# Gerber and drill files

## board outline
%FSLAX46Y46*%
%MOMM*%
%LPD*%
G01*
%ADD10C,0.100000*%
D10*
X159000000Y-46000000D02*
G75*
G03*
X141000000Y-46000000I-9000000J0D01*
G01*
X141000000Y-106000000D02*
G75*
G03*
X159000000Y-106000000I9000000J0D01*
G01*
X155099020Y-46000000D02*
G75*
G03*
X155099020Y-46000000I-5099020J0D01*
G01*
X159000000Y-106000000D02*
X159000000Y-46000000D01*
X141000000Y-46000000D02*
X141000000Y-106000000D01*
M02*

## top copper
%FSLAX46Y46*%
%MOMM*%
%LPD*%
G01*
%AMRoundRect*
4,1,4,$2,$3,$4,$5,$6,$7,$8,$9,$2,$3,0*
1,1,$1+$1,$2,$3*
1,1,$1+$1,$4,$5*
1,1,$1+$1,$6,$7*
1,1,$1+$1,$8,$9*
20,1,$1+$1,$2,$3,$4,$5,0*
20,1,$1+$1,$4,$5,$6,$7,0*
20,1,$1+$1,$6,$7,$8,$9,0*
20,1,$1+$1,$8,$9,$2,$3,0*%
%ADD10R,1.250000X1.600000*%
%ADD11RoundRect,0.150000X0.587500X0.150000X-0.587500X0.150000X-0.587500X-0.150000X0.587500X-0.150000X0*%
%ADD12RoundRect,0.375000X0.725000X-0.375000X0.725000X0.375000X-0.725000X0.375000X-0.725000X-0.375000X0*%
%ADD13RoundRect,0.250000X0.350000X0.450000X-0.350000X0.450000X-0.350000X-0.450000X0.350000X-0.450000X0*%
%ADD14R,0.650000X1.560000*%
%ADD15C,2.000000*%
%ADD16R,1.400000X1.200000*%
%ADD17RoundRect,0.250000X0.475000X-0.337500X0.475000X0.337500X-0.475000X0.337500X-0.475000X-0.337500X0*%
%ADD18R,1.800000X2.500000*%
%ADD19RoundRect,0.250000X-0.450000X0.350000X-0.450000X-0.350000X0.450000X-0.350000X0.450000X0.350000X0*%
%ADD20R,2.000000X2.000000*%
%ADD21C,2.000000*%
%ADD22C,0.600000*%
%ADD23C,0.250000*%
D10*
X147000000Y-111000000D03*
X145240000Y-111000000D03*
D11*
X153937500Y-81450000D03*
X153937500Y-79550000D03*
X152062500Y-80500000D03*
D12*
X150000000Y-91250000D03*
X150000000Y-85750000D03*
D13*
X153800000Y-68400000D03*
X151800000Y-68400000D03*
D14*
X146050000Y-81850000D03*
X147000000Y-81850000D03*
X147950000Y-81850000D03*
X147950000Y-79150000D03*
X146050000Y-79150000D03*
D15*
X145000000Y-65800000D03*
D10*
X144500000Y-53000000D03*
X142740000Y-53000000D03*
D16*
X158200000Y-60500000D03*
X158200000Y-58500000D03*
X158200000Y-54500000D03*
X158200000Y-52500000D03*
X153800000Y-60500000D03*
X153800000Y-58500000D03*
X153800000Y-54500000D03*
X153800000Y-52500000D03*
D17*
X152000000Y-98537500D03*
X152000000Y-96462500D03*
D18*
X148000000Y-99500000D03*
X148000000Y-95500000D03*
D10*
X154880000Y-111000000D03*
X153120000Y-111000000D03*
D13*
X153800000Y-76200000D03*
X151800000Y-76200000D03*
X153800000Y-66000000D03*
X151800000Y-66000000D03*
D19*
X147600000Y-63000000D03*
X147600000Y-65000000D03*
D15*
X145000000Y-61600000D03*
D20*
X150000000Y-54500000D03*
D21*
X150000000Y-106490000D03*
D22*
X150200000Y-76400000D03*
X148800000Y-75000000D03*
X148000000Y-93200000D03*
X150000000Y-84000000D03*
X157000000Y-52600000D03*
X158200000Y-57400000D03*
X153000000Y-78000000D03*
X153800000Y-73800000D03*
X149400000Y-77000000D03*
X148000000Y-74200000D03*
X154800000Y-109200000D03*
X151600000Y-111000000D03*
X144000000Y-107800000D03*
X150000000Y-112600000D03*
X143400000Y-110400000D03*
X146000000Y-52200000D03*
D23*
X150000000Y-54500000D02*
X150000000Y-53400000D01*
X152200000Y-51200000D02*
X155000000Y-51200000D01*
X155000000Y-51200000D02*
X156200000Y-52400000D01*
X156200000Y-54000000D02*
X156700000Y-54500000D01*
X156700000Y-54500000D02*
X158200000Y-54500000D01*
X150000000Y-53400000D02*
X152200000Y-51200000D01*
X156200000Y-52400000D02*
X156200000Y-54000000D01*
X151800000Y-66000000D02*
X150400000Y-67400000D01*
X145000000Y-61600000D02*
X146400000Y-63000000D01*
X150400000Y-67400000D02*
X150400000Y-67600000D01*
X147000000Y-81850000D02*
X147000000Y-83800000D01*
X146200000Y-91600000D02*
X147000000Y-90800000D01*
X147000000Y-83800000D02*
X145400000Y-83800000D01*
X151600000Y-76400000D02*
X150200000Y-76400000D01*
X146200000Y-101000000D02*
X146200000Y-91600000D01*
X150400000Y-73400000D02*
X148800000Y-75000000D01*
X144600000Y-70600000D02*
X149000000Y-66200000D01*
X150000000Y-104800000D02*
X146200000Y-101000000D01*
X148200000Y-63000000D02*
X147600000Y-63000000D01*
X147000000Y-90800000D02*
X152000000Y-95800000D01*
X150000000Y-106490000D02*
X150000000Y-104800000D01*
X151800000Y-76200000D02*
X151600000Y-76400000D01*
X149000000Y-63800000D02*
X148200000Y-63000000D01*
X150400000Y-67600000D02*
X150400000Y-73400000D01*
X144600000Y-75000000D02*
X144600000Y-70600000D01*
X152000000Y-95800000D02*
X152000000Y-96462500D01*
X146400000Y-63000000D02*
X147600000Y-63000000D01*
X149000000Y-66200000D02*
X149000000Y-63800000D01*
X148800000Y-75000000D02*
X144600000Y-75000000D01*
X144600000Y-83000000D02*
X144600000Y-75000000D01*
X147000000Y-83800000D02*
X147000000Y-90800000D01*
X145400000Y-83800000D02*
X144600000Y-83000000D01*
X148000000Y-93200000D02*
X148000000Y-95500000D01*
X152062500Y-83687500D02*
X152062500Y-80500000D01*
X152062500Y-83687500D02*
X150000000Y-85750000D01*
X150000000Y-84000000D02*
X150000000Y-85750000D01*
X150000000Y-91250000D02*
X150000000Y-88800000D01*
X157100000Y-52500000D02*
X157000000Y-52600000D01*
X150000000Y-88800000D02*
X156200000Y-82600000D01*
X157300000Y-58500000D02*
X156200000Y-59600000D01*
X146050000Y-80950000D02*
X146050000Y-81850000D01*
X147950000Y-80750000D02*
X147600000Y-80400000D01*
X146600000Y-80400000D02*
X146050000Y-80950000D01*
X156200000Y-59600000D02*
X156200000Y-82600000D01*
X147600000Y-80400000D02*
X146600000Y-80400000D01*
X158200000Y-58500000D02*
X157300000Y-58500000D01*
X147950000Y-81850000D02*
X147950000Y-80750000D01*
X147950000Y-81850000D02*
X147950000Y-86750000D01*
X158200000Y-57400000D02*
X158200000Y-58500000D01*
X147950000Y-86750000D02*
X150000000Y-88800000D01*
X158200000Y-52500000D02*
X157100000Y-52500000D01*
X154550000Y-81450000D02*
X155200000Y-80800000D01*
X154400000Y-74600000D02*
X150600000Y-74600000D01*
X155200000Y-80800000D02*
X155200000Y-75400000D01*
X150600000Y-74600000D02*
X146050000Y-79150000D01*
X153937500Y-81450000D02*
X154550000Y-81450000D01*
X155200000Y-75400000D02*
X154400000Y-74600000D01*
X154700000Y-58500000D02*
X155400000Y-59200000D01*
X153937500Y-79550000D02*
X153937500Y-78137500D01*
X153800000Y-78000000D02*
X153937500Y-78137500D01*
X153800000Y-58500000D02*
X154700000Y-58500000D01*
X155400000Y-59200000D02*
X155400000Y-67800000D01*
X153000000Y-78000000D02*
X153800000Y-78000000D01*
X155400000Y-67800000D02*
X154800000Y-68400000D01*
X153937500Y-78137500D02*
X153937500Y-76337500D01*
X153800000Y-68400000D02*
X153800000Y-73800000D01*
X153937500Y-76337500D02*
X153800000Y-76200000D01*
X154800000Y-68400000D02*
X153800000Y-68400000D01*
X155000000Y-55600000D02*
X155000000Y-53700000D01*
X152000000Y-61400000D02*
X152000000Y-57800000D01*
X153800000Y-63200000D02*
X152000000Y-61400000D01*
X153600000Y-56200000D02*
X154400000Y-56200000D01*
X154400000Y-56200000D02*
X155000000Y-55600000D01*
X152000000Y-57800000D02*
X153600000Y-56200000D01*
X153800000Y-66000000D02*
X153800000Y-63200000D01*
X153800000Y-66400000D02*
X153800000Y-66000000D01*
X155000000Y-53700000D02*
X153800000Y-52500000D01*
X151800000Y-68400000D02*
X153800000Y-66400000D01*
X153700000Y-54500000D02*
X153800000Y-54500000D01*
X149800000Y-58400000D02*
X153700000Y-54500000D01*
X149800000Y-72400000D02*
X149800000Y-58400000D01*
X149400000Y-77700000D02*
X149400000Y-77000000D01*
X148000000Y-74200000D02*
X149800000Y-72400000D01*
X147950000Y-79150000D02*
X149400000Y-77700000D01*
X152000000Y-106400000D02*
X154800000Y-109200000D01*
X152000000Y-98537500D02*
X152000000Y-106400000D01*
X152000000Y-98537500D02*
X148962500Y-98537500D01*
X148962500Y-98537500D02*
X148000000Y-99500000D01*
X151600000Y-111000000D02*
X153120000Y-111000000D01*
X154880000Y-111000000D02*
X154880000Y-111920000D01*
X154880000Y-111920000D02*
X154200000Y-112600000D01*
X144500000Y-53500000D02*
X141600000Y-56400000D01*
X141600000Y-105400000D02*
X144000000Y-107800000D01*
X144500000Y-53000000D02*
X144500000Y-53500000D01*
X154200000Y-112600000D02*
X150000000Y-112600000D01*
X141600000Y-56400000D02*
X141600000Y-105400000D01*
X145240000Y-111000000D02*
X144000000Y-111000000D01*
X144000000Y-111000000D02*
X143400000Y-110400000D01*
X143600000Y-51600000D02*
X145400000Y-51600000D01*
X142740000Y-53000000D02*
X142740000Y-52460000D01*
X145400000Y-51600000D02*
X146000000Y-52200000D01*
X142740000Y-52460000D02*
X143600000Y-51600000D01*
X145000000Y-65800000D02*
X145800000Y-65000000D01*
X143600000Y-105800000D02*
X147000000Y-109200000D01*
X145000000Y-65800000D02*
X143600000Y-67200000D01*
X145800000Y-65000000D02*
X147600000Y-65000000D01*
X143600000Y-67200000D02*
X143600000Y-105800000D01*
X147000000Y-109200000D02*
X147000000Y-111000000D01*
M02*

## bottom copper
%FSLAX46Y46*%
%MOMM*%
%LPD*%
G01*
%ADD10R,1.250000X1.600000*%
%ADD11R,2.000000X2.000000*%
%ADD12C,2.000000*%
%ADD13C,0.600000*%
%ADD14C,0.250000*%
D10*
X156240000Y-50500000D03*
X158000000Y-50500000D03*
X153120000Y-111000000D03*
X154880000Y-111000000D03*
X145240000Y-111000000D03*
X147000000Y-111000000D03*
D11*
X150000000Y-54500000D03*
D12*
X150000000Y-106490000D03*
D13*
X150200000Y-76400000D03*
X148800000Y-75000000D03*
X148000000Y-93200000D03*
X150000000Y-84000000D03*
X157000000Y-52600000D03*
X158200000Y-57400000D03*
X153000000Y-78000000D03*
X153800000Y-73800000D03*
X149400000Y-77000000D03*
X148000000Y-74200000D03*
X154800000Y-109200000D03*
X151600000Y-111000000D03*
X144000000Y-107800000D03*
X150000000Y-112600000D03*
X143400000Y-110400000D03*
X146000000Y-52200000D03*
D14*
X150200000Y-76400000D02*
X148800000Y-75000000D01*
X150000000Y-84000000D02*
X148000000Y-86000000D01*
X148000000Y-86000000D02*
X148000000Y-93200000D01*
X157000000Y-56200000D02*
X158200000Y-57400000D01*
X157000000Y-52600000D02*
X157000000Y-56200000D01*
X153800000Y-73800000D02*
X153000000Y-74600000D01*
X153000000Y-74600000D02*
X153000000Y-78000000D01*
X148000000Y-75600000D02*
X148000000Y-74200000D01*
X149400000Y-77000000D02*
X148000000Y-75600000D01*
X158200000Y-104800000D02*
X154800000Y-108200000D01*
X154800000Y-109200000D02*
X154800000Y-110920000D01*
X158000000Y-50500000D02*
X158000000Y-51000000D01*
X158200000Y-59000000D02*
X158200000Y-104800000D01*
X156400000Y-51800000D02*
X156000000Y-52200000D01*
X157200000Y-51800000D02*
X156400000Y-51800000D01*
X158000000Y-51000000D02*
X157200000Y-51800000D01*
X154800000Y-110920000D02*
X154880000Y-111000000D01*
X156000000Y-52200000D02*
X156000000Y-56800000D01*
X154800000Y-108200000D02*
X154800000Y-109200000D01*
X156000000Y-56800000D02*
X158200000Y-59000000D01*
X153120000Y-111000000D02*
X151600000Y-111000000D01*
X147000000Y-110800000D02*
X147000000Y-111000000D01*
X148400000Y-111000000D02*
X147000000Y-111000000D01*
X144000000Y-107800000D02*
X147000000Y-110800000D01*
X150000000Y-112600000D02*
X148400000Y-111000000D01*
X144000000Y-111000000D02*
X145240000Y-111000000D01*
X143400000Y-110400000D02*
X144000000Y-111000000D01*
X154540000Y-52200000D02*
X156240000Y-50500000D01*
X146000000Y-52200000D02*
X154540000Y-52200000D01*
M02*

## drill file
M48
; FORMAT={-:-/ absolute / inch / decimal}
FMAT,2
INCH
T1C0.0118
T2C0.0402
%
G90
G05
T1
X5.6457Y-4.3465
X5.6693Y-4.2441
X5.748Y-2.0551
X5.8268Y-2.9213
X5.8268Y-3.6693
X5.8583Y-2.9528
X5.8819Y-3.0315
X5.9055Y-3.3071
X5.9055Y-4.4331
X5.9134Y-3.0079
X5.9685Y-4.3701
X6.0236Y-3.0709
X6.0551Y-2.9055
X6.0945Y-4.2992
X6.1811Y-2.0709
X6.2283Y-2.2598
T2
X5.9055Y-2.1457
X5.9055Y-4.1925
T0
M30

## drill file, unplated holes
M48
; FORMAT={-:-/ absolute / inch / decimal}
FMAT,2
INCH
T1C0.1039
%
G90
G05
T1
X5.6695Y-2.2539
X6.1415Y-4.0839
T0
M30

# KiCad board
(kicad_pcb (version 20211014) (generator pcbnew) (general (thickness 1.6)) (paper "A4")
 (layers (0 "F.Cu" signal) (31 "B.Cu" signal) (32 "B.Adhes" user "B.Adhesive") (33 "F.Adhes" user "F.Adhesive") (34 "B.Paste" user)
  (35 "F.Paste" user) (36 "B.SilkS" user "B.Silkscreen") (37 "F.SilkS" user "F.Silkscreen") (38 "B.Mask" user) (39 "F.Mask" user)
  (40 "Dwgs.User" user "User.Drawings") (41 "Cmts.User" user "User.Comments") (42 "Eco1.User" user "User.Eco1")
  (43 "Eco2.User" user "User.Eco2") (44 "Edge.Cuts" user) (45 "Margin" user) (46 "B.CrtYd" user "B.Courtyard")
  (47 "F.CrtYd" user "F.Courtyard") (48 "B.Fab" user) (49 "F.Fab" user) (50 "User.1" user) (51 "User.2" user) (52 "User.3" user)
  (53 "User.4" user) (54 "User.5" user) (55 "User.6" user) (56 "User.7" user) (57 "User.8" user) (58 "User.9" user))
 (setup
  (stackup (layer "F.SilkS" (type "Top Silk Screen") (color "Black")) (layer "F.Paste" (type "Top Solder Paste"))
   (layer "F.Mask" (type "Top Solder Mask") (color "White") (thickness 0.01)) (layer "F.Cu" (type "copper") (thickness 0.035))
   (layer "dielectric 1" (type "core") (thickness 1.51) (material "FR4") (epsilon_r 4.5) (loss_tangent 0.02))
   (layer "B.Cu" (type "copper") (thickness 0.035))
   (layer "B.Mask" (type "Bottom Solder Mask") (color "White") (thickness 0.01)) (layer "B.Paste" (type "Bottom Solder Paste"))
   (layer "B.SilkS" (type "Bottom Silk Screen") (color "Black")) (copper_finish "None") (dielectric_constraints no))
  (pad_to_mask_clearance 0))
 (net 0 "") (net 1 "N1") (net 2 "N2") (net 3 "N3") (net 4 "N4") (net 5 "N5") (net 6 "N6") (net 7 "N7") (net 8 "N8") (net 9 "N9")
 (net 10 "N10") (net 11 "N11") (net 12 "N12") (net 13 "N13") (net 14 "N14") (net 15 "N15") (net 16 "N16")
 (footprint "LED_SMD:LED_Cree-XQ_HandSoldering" (layer "F.Cu") (at 146.12 111 180)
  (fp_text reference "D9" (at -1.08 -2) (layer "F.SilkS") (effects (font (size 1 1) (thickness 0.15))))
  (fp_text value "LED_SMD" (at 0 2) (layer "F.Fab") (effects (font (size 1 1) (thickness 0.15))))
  (pad "1" smd rect (at -0.88 0 180) (size 1.25 1.6) (layers "F.Cu" "F.Paste" "F.Mask") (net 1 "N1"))
  (pad "2" smd rect (at 0.88 0 180) (size 1.25 1.6) (layers "F.Cu" "F.Paste" "F.Mask") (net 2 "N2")))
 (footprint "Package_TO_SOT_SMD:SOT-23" (layer "F.Cu") (at 153 80.5 180)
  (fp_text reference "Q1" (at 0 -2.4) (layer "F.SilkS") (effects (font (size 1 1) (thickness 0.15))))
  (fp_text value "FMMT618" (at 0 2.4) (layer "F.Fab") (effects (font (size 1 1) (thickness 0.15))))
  (pad "1" smd roundrect (at -0.9375 -0.95 180) (size 1.475 0.6) (layers "F.Cu" "F.Paste" "F.Mask") (roundrect_rratio 0.25) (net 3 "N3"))
  (pad "2" smd roundrect (at -0.9375 0.95 180) (size 1.475 0.6) (layers "F.Cu" "F.Paste" "F.Mask") (roundrect_rratio 0.25) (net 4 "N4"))
  (pad "3" smd roundrect (at 0.9375 0 180) (size 1.475 0.6) (layers "F.Cu" "F.Paste" "F.Mask") (roundrect_rratio 0.25) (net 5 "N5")))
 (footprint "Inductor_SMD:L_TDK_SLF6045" (layer "F.Cu") (at 150 88.5 90)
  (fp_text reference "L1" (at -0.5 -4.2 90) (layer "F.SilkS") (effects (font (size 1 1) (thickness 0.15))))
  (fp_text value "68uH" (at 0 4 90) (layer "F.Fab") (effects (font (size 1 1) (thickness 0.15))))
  (pad "1" smd roundrect (at -2.75 0 90) (size 1.5 2.2) (layers "F.Cu" "F.Paste" "F.Mask") (roundrect_rratio 0.25) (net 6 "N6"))
  (pad "2" smd roundrect (at 2.75 0 90) (size 1.5 2.2) (layers "F.Cu" "F.Paste" "F.Mask") (roundrect_rratio 0.25) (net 5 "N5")))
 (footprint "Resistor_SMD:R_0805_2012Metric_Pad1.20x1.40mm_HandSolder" (layer "F.Cu") (at 152.8 68.4 180)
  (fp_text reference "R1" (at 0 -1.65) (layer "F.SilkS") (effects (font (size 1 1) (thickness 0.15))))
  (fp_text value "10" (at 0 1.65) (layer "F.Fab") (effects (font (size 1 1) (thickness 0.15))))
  (pad "1" smd roundrect (at -1 0 180) (size 1.2 1.4) (layers "F.Cu" "F.Paste" "F.Mask") (roundrect_rratio 0.2083333333) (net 4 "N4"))
  (pad "2" smd roundrect (at 1 0 180) (size 1.2 1.4) (layers "F.Cu" "F.Paste" "F.Mask") (roundrect_rratio 0.2083333333) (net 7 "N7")))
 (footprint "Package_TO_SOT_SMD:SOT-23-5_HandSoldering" (layer "F.Cu") (at 147 80.5 90)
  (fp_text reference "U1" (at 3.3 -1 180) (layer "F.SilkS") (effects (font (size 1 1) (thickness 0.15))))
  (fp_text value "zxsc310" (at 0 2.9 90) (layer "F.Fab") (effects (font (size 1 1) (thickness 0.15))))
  (pad "1" smd rect (at -1.35 -0.95 90) (size 1.56 0.65) (layers "F.Cu" "F.Paste" "F.Mask") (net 6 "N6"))
  (pad "2" smd rect (at -1.35 0 90) (size 1.56 0.65) (layers "F.Cu" "F.Paste" "F.Mask") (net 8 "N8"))
  (pad "3" smd rect (at -1.35 0.95 90) (size 1.56 0.65) (layers "F.Cu" "F.Paste" "F.Mask") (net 6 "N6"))
  (pad "4" smd rect (at 1.35 0.95 90) (size 1.56 0.65) (layers "F.Cu" "F.Paste" "F.Mask") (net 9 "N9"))
  (pad "5" smd rect (at 1.35 -0.95 90) (size 1.56 0.65) (layers "F.Cu" "F.Paste" "F.Mask") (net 3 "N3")))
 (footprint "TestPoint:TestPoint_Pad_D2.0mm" (layer "F.Cu") (at 145 65.8)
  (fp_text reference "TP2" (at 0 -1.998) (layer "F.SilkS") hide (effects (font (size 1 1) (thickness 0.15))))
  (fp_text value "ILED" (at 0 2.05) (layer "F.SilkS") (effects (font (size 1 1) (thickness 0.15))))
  (pad "1" smd circle (at 0 0) (size 2 2) (layers "F.Cu" "F.Mask") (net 1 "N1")))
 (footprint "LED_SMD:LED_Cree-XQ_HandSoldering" (layer "F.Cu") (at 143.62 53 180)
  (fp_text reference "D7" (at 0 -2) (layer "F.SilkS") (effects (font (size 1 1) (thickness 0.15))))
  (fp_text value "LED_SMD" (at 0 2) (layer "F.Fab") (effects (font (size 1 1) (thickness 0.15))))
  (pad "1" smd rect (at -0.88 0 180) (size 1.25 1.6) (layers "F.Cu" "F.Paste" "F.Mask") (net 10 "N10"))
  (pad "2" smd rect (at 0.88 0 180) (size 1.25 1.6) (layers "F.Cu" "F.Paste" "F.Mask") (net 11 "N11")))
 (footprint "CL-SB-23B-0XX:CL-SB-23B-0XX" (layer "F.Cu") (at 156 56.5 90)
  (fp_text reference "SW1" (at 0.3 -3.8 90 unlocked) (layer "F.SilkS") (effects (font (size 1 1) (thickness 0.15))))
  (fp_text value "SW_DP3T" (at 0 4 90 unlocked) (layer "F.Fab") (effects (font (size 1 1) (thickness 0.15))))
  (pad "1" smd rect (at -4 2.2 90) (size 1.2 1.4) (layers "F.Cu" "F.Paste" "F.Mask") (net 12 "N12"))
  (pad "2" smd rect (at -2 2.2 90) (size 1.2 1.4) (layers "F.Cu" "F.Paste" "F.Mask") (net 6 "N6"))
  (pad "3" smd rect (at 2 2.2 90) (size 1.2 1.4) (layers "F.Cu" "F.Paste" "F.Mask") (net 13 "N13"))
  (pad "4" smd rect (at 4 2.2 90) (size 1.2 1.4) (layers "F.Cu" "F.Paste" "F.Mask") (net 6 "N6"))
  (pad "5" smd rect (at -4 -2.2 90) (size 1.2 1.4) (layers "F.Cu" "F.Paste" "F.Mask") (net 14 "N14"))
  (pad "6" smd rect (at -2 -2.2 90) (size 1.2 1.4) (layers "F.Cu" "F.Paste" "F.Mask") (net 4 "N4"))
  (pad "7" smd rect (at 2 -2.2 90) (size 1.2 1.4) (layers "F.Cu" "F.Paste" "F.Mask") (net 9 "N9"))
  (pad "8" smd rect (at 4 -2.2 90) (size 1.2 1.4) (layers "F.Cu" "F.Paste" "F.Mask") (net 7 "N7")))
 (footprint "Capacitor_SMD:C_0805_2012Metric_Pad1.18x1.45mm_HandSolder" (layer "F.Cu") (at 152 97.5 90)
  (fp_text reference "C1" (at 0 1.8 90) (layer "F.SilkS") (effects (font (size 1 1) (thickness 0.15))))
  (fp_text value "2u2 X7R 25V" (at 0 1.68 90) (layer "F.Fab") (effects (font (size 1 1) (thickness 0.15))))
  (pad "1" smd roundrect (at -1.0375 0 90) (size 1.175 1.45) (layers "F.Cu" "F.Paste" "F.Mask") (roundrect_rratio 0.2127659574)
   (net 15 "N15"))
  (pad "2" smd roundrect (at 1.0375 0 90) (size 1.175 1.45) (layers "F.Cu" "F.Paste" "F.Mask") (roundrect_rratio 0.2127659574) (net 8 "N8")))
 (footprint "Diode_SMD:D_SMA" (layer "F.Cu") (at 148 97.5 90)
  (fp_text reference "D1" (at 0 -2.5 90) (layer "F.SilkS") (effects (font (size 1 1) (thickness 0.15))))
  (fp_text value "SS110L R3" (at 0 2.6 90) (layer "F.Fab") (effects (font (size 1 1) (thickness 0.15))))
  (pad "1" smd rect (at -2 0 90) (size 2.5 1.8) (layers "F.Cu" "F.Paste" "F.Mask") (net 15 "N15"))
  (pad "2" smd rect (at 2 0 90) (size 2.5 1.8) (layers "F.Cu" "F.Paste" "F.Mask") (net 5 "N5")))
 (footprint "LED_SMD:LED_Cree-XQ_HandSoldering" (layer "F.Cu") (at 154 111 180)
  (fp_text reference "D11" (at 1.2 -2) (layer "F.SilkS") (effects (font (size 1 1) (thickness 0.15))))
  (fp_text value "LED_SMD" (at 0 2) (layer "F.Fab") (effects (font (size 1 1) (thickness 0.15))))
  (pad "1" smd rect (at -0.88 0 180) (size 1.25 1.6) (layers "F.Cu" "F.Paste" "F.Mask") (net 10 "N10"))
  (pad "2" smd rect (at 0.88 0 180) (size 1.25 1.6) (layers "F.Cu" "F.Paste" "F.Mask") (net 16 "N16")))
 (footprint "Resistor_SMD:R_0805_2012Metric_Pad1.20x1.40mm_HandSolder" (layer "F.Cu") (at 152.8 76.2 180)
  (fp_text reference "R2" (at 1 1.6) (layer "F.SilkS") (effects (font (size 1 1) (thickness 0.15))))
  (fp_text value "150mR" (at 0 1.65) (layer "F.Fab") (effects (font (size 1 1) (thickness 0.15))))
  (pad "1" smd roundrect (at -1 0 180) (size 1.2 1.4) (layers "F.Cu" "F.Paste" "F.Mask") (roundrect_rratio 0.2083333333) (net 4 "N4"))
  (pad "2" smd roundrect (at 1 0 180) (size 1.2 1.4) (layers "F.Cu" "F.Paste" "F.Mask") (roundrect_rratio 0.2083333333) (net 8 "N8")))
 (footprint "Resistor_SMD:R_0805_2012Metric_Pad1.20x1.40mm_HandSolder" (layer "F.Cu") (at 152.8 66 180)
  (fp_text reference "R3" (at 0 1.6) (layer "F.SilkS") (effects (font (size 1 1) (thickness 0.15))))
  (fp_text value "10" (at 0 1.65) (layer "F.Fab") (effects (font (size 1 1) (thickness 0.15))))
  (pad "1" smd roundrect (at -1 0 180) (size 1.2 1.4) (layers "F.Cu" "F.Paste" "F.Mask") (roundrect_rratio 0.2083333333) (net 7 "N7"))
  (pad "2" smd roundrect (at 1 0 180) (size 1.2 1.4) (layers "F.Cu" "F.Paste" "F.Mask") (roundrect_rratio 0.2083333333) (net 8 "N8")))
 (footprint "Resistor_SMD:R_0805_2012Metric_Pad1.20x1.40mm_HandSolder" (layer "F.Cu") (at 147.6 64 -90)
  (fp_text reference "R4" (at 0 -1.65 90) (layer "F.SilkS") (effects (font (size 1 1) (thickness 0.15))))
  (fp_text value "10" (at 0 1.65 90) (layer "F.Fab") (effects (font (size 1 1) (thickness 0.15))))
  (pad "1" smd roundrect (at -1 0 270) (size 1.2 1.4) (layers "F.Cu" "F.Paste" "F.Mask") (roundrect_rratio 0.2083333333) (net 8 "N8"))
  (pad "2" smd roundrect (at 1 0 270) (size 1.2 1.4) (layers "F.Cu" "F.Paste" "F.Mask") (roundrect_rratio 0.2083333333) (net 1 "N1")))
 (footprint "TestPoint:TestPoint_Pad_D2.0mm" (layer "F.Cu") (at 145 61.6)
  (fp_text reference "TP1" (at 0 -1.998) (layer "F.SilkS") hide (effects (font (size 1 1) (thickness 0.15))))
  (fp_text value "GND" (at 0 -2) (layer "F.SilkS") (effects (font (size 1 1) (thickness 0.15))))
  (pad "1" smd circle (at 0 0) (size 2 2) (layers "F.Cu" "F.Mask") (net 8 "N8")))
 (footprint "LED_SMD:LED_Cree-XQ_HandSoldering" (layer "B.Cu") (at 157.12 50.5)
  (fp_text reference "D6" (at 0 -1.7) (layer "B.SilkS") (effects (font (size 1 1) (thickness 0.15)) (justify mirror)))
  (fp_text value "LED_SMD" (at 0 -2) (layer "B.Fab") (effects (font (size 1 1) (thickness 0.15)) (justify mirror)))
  (pad "1" smd rect (at -0.88 0) (size 1.25 1.6) (layers "B.Cu" "B.Paste" "B.Mask") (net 11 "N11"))
  (pad "2" smd rect (at 0.88 0) (size 1.25 1.6) (layers "B.Cu" "B.Paste" "B.Mask") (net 15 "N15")))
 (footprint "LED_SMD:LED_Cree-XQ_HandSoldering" (layer "B.Cu") (at 154 111)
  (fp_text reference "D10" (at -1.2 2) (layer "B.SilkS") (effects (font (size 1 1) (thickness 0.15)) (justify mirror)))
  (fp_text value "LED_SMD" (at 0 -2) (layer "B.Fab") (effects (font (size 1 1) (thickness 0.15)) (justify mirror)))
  (pad "1" smd rect (at -0.88 0) (size 1.25 1.6) (layers "B.Cu" "B.Paste" "B.Mask") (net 16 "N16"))
  (pad "2" smd rect (at 0.88 0) (size 1.25 1.6) (layers "B.Cu" "B.Paste" "B.Mask") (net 15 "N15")))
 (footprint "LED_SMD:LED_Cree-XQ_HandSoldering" (layer "B.Cu") (at 146.12 111)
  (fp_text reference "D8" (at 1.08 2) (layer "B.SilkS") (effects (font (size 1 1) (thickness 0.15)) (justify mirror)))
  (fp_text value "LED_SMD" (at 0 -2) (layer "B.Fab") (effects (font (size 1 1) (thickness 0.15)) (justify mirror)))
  (pad "1" smd rect (at -0.88 0) (size 1.25 1.6) (layers "B.Cu" "B.Paste" "B.Mask") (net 2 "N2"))
  (pad "2" smd rect (at 0.88 0) (size 1.25 1.6) (layers "B.Cu" "B.Paste" "B.Mask") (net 10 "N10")))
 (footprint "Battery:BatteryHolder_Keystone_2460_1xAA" (layer "B.Cu") (at 150 54.5 -90)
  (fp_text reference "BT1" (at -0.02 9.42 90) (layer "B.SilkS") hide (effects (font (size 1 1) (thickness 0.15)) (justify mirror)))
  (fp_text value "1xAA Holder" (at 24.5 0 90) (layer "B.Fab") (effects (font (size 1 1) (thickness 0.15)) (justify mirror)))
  (pad "" np_thru_hole circle (at 49.23 -5.995 270) (size 2.64 2.64) (drill 2.64) (layers *.Cu *.Mask))
  (pad "" np_thru_hole circle (at 2.75 5.995 180) (size 2.64 2.64) (drill 2.64) (layers *.Cu *.Mask))
  (pad "1" thru_hole rect (at 0 0 90) (size 2 2) (drill 1.02) (layers *.Cu *.Mask) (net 13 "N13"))
  (pad "2" thru_hole circle (at 51.99 0 90) (size 2 2) (drill 1.02) (layers *.Cu *.Mask) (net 8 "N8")))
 (gr_arc (start 141 46) (mid 150 37) (end 159 46) (layer "Edge.Cuts") (width 0.1))
 (gr_arc (start 159 106) (mid 150 115) (end 141 106) (layer "Edge.Cuts") (width 0.1))
 (gr_circle (center 150 46) (end 155 45) (layer "Edge.Cuts") (width 0.1) (fill none))
 (gr_line (start 159 106) (end 159 46) (layer "Edge.Cuts") (width 0.1))
 (gr_line (start 141 46) (end 141 106) (layer "Edge.Cuts") (width 0.1))
 (segment (start 150 54.5) (end 150 53.4) (width 0.25) (layer "F.Cu") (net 13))
 (segment (start 152.2 51.2) (end 155 51.2) (width 0.25) (layer "F.Cu") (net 13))
 (segment (start 155 51.2) (end 156.2 52.4) (width 0.25) (layer "F.Cu") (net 13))
 (segment (start 156.2 54) (end 156.7 54.5) (width 0.25) (layer "F.Cu") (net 13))
 (segment (start 156.7 54.5) (end 158.2 54.5) (width 0.25) (layer "F.Cu") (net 13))
 (segment (start 150 53.4) (end 152.2 51.2) (width 0.25) (layer "F.Cu") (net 13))
 (segment (start 156.2 52.4) (end 156.2 54) (width 0.25) (layer "F.Cu") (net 13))
 (segment (start 151.8 66) (end 150.4 67.4) (width 0.25) (layer "F.Cu") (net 8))
 (segment (start 145 61.6) (end 146.4 63) (width 0.25) (layer "F.Cu") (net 8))
 (segment (start 150.4 67.4) (end 150.4 67.6) (width 0.25) (layer "F.Cu") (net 8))
 (segment (start 147 81.85) (end 147 83.8) (width 0.25) (layer "F.Cu") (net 8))
 (segment (start 146.2 91.6) (end 147 90.8) (width 0.25) (layer "F.Cu") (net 8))
 (segment (start 147 83.8) (end 145.4 83.8) (width 0.25) (layer "F.Cu") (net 8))
 (segment (start 151.6 76.4) (end 150.2 76.4) (width 0.25) (layer "F.Cu") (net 8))
 (segment (start 146.2 101) (end 146.2 91.6) (width 0.25) (layer "F.Cu") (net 8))
 (segment (start 150.4 73.4) (end 148.8 75) (width 0.25) (layer "F.Cu") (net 8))
 (segment (start 144.6 70.6) (end 149 66.2) (width 0.25) (layer "F.Cu") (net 8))
 (segment (start 150 104.8) (end 146.2 101) (width 0.25) (layer "F.Cu") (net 8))
 (segment (start 148.2 63) (end 147.6 63) (width 0.25) (layer "F.Cu") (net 8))
 (segment (start 147 90.8) (end 152 95.8) (width 0.25) (layer "F.Cu") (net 8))
 (segment (start 150 106.49) (end 150 104.8) (width 0.25) (layer "F.Cu") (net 8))
 (segment (start 151.8 76.2) (end 151.6 76.4) (width 0.25) (layer "F.Cu") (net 8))
 (segment (start 149 63.8) (end 148.2 63) (width 0.25) (layer "F.Cu") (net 8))
 (segment (start 150.4 67.6) (end 150.4 73.4) (width 0.25) (layer "F.Cu") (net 8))
 (segment (start 144.6 75) (end 144.6 70.6) (width 0.25) (layer "F.Cu") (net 8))
 (segment (start 152 95.8) (end 152 96.4625) (width 0.25) (layer "F.Cu") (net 8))
 (segment (start 146.4 63) (end 147.6 63) (width 0.25) (layer "F.Cu") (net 8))
 (segment (start 149 66.2) (end 149 63.8) (width 0.25) (layer "F.Cu") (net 8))
 (segment (start 148.8 75) (end 144.6 75) (width 0.25) (layer "F.Cu") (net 8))
 (segment (start 144.6 83) (end 144.6 75) (width 0.25) (layer "F.Cu") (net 8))
 (segment (start 147 83.8) (end 147 90.8) (width 0.25) (layer "F.Cu") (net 8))
 (segment (start 145.4 83.8) (end 144.6 83) (width 0.25) (layer "F.Cu") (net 8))
 (via (at 150.2 76.4) (size 0.6) (drill 0.3) (layers "F.Cu" "B.Cu") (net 8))
 (via (at 148.8 75) (size 0.6) (drill 0.3) (layers "F.Cu" "B.Cu") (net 8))
 (segment (start 150.2 76.4) (end 148.8 75) (width 0.25) (layer "B.Cu") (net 8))
 (segment (start 148 93.2) (end 148 95.5) (width 0.25) (layer "F.Cu") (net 5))
 (segment (start 152.0625 83.6875) (end 152.0625 80.5) (width 0.25) (layer "F.Cu") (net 5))
 (segment (start 152.0625 83.6875) (end 150 85.75) (width 0.25) (layer "F.Cu") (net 5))
 (segment (start 150 84) (end 150 85.75) (width 0.25) (layer "F.Cu") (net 5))
 (via (at 148 93.2) (size 0.6) (drill 0.3) (layers "F.Cu" "B.Cu") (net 5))
 (via (at 150 84) (size 0.6) (drill 0.3) (layers "F.Cu" "B.Cu") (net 5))
 (segment (start 150 84) (end 148 86) (width 0.25) (layer "B.Cu") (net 5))
 (segment (start 148 86) (end 148 93.2) (width 0.25) (layer "B.Cu") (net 5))
 (segment (start 150 91.25) (end 150 88.8) (width 0.25) (layer "F.Cu") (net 6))
 (segment (start 157.1 52.5) (end 157 52.6) (width 0.25) (layer "F.Cu") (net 6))
 (segment (start 150 88.8) (end 156.2 82.6) (width 0.25) (layer "F.Cu") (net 6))
 (segment (start 157.3 58.5) (end 156.2 59.6) (width 0.25) (layer "F.Cu") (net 6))
 (segment (start 146.05 80.95) (end 146.05 81.85) (width 0.25) (layer "F.Cu") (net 6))
 (segment (start 147.95 80.75) (end 147.6 80.4) (width 0.25) (layer "F.Cu") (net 6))
 (segment (start 146.6 80.4) (end 146.05 80.95) (width 0.25) (layer "F.Cu") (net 6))
 (segment (start 156.2 59.6) (end 156.2 82.6) (width 0.25) (layer "F.Cu") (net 6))
 (segment (start 147.6 80.4) (end 146.6 80.4) (width 0.25) (layer "F.Cu") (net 6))
 (segment (start 158.2 58.5) (end 157.3 58.5) (width 0.25) (layer "F.Cu") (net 6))
 (segment (start 147.95 81.85) (end 147.95 80.75) (width 0.25) (layer "F.Cu") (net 6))
 (segment (start 147.95 81.85) (end 147.95 86.75) (width 0.25) (layer "F.Cu") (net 6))
 (segment (start 158.2 57.4) (end 158.2 58.5) (width 0.25) (layer "F.Cu") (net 6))
 (segment (start 147.95 86.75) (end 150 88.8) (width 0.25) (layer "F.Cu") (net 6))
 (segment (start 158.2 52.5) (end 157.1 52.5) (width 0.25) (layer "F.Cu") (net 6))
 (via (at 157 52.6) (size 0.6) (drill 0.3) (layers "F.Cu" "B.Cu") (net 6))
 (via (at 158.2 57.4) (size 0.6) (drill 0.3) (layers "F.Cu" "B.Cu") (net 6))
 (segment (start 157 56.2) (end 158.2 57.4) (width 0.25) (layer "B.Cu") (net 6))
 (segment (start 157 52.6) (end 157 56.2) (width 0.25) (layer "B.Cu") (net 6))
 (segment (start 154.55 81.45) (end 155.2 80.8) (width 0.25) (layer "F.Cu") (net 3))
 (segment (start 154.4 74.6) (end 150.6 74.6) (width 0.25) (layer "F.Cu") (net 3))
 (segment (start 155.2 80.8) (end 155.2 75.4) (width 0.25) (layer "F.Cu") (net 3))
 (segment (start 150.6 74.6) (end 146.05 79.15) (width 0.25) (layer "F.Cu") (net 3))
 (segment (start 153.9375 81.45) (end 154.55 81.45) (width 0.25) (layer "F.Cu") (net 3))
 (segment (start 155.2 75.4) (end 154.4 74.6) (width 0.25) (layer "F.Cu") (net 3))
 (segment (start 154.7 58.5) (end 155.4 59.2) (width 0.25) (layer "F.Cu") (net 4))
 (segment (start 153.9375 79.55) (end 153.9375 78.1375) (width 0.25) (layer "F.Cu") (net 4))
 (segment (start 153.8 78) (end 153.9375 78.1375) (width 0.25) (layer "F.Cu") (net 4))
 (segment (start 153.8 58.5) (end 154.7 58.5) (width 0.25) (layer "F.Cu") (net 4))
 (segment (start 155.4 59.2) (end 155.4 67.8) (width 0.25) (layer "F.Cu") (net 4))
 (segment (start 153 78) (end 153.8 78) (width 0.25) (layer "F.Cu") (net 4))
 (segment (start 155.4 67.8) (end 154.8 68.4) (width 0.25) (layer "F.Cu") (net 4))
 (segment (start 153.9375 78.1375) (end 153.9375 76.3375) (width 0.25) (layer "F.Cu") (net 4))
 (segment (start 153.8 68.4) (end 153.8 73.8) (width 0.25) (layer "F.Cu") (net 4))
 (segment (start 153.9375 76.3375) (end 153.8 76.2) (width 0.25) (layer "F.Cu") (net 4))
 (segment (start 154.8 68.4) (end 153.8 68.4) (width 0.25) (layer "F.Cu") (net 4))
 (via (at 153 78) (size 0.6) (drill 0.3) (layers "F.Cu" "B.Cu") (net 4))
 (via (at 153.8 73.8) (size 0.6) (drill 0.3) (layers "F.Cu" "B.Cu") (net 4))
 (segment (start 153.8 73.8) (end 153 74.6) (width 0.25) (layer "B.Cu") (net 4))
 (segment (start 153 74.6) (end 153 78) (width 0.25) (layer "B.Cu") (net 4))
 (segment (start 155 55.6) (end 155 53.7) (width 0.25) (layer "F.Cu") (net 7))
 (segment (start 152 61.4) (end 152 57.8) (width 0.25) (layer "F.Cu") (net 7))
 (segment (start 153.8 63.2) (end 152 61.4) (width 0.25) (layer "F.Cu") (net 7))
 (segment (start 153.6 56.2) (end 154.4 56.2) (width 0.25) (layer "F.Cu") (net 7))
 (segment (start 154.4 56.2) (end 155 55.6) (width 0.25) (layer "F.Cu") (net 7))
 (segment (start 152 57.8) (end 153.6 56.2) (width 0.25) (layer "F.Cu") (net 7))
 (segment (start 153.8 66) (end 153.8 63.2) (width 0.25) (layer "F.Cu") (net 7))
 (segment (start 153.8 66.4) (end 153.8 66) (width 0.25) (layer "F.Cu") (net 7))
 (segment (start 155 53.7) (end 153.8 52.5) (width 0.25) (layer "F.Cu") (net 7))
 (segment (start 151.8 68.4) (end 153.8 66.4) (width 0.25) (layer "F.Cu") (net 7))
 (segment (start 153.7 54.5) (end 153.8 54.5) (width 0.25) (layer "F.Cu") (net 9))
 (segment (start 149.8 58.4) (end 153.7 54.5) (width 0.25) (layer "F.Cu") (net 9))
 (segment (start 149.8 72.4) (end 149.8 58.4) (width 0.25) (layer "F.Cu") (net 9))
 (segment (start 149.4 77.7) (end 149.4 77) (width 0.25) (layer "F.Cu") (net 9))
 (segment (start 148 74.2) (end 149.8 72.4) (width 0.25) (layer "F.Cu") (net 9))
 (segment (start 147.95 79.15) (end 149.4 77.7) (width 0.25) (layer "F.Cu") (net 9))
 (via (at 149.4 77) (size 0.6) (drill 0.3) (layers "F.Cu" "B.Cu") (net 9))
 (via (at 148 74.2) (size 0.6) (drill 0.3) (layers "F.Cu" "B.Cu") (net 9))
 (segment (start 148 75.6) (end 148 74.2) (width 0.25) (layer "B.Cu") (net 9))
 (segment (start 149.4 77) (end 148 75.6) (width 0.25) (layer "B.Cu") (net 9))
 (segment (start 152 106.4) (end 154.8 109.2) (width 0.25) (layer "F.Cu") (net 15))
 (segment (start 152 98.5375) (end 152 106.4) (width 0.25) (layer "F.Cu") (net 15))
 (segment (start 152 98.5375) (end 148.9625 98.5375) (width 0.25) (layer "F.Cu") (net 15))
 (segment (start 148.9625 98.5375) (end 148 99.5) (width 0.25) (layer "F.Cu") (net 15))
 (via (at 154.8 109.2) (size 0.6) (drill 0.3) (layers "F.Cu" "B.Cu") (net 15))
 (segment (start 158.2 104.8) (end 154.8 108.2) (width 0.25) (layer "B.Cu") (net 15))
 (segment (start 154.8 109.2) (end 154.8 110.92) (width 0.25) (layer "B.Cu") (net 15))
 (segment (start 158 50.5) (end 158 51) (width 0.25) (layer "B.Cu") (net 15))
 (segment (start 158.2 59) (end 158.2 104.8) (width 0.25) (layer "B.Cu") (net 15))
 (segment (start 156.4 51.8) (end 156 52.2) (width 0.25) (layer "B.Cu") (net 15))
 (segment (start 157.2 51.8) (end 156.4 51.8) (width 0.25) (layer "B.Cu") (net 15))
 (segment (start 158 51) (end 157.2 51.8) (width 0.25) (layer "B.Cu") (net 15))
 (segment (start 154.8 110.92) (end 154.88 111) (width 0.25) (layer "B.Cu") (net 15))
 (segment (start 156 52.2) (end 156 56.8) (width 0.25) (layer "B.Cu") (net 15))
 (segment (start 154.8 108.2) (end 154.8 109.2) (width 0.25) (layer "B.Cu") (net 15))
 (segment (start 156 56.8) (end 158.2 59) (width 0.25) (layer "B.Cu") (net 15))
 (segment (start 151.6 111) (end 153.12 111) (width 0.25) (layer "F.Cu") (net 16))
 (via (at 151.6 111) (size 0.6) (drill 0.3) (layers "F.Cu" "B.Cu") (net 16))
 (segment (start 153.12 111) (end 151.6 111) (width 0.25) (layer "B.Cu") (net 16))
 (segment (start 154.88 111) (end 154.88 111.92) (width 0.25) (layer "F.Cu") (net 10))
 (segment (start 154.88 111.92) (end 154.2 112.6) (width 0.25) (layer "F.Cu") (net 10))
 (segment (start 144.5 53.5) (end 141.6 56.4) (width 0.25) (layer "F.Cu") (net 10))
 (segment (start 141.6 105.4) (end 144 107.8) (width 0.25) (layer "F.Cu") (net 10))
 (segment (start 144.5 53) (end 144.5 53.5) (width 0.25) (layer "F.Cu") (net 10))
 (segment (start 154.2 112.6) (end 150 112.6) (width 0.25) (layer "F.Cu") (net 10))
 (segment (start 141.6 56.4) (end 141.6 105.4) (width 0.25) (layer "F.Cu") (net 10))
 (via (at 144 107.8) (size 0.6) (drill 0.3) (layers "F.Cu" "B.Cu") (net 10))
 (via (at 150 112.6) (size 0.6) (drill 0.3) (layers "F.Cu" "B.Cu") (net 10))
 (segment (start 147 110.8) (end 147 111) (width 0.25) (layer "B.Cu") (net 10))
 (segment (start 148.4 111) (end 147 111) (width 0.25) (layer "B.Cu") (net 10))
 (segment (start 144 107.8) (end 147 110.8) (width 0.25) (layer "B.Cu") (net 10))
 (segment (start 150 112.6) (end 148.4 111) (width 0.25) (layer "B.Cu") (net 10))
 (segment (start 145.24 111) (end 144 111) (width 0.25) (layer "F.Cu") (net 2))
 (segment (start 144 111) (end 143.4 110.4) (width 0.25) (layer "F.Cu") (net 2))
 (via (at 143.4 110.4) (size 0.6) (drill 0.3) (layers "F.Cu" "B.Cu") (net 2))
 (segment (start 144 111) (end 145.24 111) (width 0.25) (layer "B.Cu") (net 2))
 (segment (start 143.4 110.4) (end 144 111) (width 0.25) (layer "B.Cu") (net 2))
 (segment (start 143.6 51.6) (end 145.4 51.6) (width 0.25) (layer "F.Cu") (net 11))
 (segment (start 142.74 53) (end 142.74 52.46) (width 0.25) (layer "F.Cu") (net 11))
 (segment (start 145.4 51.6) (end 146 52.2) (width 0.25) (layer "F.Cu") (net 11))
 (segment (start 142.74 52.46) (end 143.6 51.6) (width 0.25) (layer "F.Cu") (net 11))
 (via (at 146 52.2) (size 0.6) (drill 0.3) (layers "F.Cu" "B.Cu") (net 11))
 (segment (start 154.54 52.2) (end 156.24 50.5) (width 0.25) (layer "B.Cu") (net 11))
 (segment (start 146 52.2) (end 154.54 52.2) (width 0.25) (layer "B.Cu") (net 11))
 (segment (start 145 65.8) (end 145.8 65) (width 0.25) (layer "F.Cu") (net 1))
 (segment (start 143.6 105.8) (end 147 109.2) (width 0.25) (layer "F.Cu") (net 1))
 (segment (start 145 65.8) (end 143.6 67.2) (width 0.25) (layer "F.Cu") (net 1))
 (segment (start 145.8 65) (end 147.6 65) (width 0.25) (layer "F.Cu") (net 1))
 (segment (start 143.6 67.2) (end 143.6 105.8) (width 0.25) (layer "F.Cu") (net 1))
 (segment (start 147 109.2) (end 147 111) (width 0.25) (layer "F.Cu") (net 1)))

